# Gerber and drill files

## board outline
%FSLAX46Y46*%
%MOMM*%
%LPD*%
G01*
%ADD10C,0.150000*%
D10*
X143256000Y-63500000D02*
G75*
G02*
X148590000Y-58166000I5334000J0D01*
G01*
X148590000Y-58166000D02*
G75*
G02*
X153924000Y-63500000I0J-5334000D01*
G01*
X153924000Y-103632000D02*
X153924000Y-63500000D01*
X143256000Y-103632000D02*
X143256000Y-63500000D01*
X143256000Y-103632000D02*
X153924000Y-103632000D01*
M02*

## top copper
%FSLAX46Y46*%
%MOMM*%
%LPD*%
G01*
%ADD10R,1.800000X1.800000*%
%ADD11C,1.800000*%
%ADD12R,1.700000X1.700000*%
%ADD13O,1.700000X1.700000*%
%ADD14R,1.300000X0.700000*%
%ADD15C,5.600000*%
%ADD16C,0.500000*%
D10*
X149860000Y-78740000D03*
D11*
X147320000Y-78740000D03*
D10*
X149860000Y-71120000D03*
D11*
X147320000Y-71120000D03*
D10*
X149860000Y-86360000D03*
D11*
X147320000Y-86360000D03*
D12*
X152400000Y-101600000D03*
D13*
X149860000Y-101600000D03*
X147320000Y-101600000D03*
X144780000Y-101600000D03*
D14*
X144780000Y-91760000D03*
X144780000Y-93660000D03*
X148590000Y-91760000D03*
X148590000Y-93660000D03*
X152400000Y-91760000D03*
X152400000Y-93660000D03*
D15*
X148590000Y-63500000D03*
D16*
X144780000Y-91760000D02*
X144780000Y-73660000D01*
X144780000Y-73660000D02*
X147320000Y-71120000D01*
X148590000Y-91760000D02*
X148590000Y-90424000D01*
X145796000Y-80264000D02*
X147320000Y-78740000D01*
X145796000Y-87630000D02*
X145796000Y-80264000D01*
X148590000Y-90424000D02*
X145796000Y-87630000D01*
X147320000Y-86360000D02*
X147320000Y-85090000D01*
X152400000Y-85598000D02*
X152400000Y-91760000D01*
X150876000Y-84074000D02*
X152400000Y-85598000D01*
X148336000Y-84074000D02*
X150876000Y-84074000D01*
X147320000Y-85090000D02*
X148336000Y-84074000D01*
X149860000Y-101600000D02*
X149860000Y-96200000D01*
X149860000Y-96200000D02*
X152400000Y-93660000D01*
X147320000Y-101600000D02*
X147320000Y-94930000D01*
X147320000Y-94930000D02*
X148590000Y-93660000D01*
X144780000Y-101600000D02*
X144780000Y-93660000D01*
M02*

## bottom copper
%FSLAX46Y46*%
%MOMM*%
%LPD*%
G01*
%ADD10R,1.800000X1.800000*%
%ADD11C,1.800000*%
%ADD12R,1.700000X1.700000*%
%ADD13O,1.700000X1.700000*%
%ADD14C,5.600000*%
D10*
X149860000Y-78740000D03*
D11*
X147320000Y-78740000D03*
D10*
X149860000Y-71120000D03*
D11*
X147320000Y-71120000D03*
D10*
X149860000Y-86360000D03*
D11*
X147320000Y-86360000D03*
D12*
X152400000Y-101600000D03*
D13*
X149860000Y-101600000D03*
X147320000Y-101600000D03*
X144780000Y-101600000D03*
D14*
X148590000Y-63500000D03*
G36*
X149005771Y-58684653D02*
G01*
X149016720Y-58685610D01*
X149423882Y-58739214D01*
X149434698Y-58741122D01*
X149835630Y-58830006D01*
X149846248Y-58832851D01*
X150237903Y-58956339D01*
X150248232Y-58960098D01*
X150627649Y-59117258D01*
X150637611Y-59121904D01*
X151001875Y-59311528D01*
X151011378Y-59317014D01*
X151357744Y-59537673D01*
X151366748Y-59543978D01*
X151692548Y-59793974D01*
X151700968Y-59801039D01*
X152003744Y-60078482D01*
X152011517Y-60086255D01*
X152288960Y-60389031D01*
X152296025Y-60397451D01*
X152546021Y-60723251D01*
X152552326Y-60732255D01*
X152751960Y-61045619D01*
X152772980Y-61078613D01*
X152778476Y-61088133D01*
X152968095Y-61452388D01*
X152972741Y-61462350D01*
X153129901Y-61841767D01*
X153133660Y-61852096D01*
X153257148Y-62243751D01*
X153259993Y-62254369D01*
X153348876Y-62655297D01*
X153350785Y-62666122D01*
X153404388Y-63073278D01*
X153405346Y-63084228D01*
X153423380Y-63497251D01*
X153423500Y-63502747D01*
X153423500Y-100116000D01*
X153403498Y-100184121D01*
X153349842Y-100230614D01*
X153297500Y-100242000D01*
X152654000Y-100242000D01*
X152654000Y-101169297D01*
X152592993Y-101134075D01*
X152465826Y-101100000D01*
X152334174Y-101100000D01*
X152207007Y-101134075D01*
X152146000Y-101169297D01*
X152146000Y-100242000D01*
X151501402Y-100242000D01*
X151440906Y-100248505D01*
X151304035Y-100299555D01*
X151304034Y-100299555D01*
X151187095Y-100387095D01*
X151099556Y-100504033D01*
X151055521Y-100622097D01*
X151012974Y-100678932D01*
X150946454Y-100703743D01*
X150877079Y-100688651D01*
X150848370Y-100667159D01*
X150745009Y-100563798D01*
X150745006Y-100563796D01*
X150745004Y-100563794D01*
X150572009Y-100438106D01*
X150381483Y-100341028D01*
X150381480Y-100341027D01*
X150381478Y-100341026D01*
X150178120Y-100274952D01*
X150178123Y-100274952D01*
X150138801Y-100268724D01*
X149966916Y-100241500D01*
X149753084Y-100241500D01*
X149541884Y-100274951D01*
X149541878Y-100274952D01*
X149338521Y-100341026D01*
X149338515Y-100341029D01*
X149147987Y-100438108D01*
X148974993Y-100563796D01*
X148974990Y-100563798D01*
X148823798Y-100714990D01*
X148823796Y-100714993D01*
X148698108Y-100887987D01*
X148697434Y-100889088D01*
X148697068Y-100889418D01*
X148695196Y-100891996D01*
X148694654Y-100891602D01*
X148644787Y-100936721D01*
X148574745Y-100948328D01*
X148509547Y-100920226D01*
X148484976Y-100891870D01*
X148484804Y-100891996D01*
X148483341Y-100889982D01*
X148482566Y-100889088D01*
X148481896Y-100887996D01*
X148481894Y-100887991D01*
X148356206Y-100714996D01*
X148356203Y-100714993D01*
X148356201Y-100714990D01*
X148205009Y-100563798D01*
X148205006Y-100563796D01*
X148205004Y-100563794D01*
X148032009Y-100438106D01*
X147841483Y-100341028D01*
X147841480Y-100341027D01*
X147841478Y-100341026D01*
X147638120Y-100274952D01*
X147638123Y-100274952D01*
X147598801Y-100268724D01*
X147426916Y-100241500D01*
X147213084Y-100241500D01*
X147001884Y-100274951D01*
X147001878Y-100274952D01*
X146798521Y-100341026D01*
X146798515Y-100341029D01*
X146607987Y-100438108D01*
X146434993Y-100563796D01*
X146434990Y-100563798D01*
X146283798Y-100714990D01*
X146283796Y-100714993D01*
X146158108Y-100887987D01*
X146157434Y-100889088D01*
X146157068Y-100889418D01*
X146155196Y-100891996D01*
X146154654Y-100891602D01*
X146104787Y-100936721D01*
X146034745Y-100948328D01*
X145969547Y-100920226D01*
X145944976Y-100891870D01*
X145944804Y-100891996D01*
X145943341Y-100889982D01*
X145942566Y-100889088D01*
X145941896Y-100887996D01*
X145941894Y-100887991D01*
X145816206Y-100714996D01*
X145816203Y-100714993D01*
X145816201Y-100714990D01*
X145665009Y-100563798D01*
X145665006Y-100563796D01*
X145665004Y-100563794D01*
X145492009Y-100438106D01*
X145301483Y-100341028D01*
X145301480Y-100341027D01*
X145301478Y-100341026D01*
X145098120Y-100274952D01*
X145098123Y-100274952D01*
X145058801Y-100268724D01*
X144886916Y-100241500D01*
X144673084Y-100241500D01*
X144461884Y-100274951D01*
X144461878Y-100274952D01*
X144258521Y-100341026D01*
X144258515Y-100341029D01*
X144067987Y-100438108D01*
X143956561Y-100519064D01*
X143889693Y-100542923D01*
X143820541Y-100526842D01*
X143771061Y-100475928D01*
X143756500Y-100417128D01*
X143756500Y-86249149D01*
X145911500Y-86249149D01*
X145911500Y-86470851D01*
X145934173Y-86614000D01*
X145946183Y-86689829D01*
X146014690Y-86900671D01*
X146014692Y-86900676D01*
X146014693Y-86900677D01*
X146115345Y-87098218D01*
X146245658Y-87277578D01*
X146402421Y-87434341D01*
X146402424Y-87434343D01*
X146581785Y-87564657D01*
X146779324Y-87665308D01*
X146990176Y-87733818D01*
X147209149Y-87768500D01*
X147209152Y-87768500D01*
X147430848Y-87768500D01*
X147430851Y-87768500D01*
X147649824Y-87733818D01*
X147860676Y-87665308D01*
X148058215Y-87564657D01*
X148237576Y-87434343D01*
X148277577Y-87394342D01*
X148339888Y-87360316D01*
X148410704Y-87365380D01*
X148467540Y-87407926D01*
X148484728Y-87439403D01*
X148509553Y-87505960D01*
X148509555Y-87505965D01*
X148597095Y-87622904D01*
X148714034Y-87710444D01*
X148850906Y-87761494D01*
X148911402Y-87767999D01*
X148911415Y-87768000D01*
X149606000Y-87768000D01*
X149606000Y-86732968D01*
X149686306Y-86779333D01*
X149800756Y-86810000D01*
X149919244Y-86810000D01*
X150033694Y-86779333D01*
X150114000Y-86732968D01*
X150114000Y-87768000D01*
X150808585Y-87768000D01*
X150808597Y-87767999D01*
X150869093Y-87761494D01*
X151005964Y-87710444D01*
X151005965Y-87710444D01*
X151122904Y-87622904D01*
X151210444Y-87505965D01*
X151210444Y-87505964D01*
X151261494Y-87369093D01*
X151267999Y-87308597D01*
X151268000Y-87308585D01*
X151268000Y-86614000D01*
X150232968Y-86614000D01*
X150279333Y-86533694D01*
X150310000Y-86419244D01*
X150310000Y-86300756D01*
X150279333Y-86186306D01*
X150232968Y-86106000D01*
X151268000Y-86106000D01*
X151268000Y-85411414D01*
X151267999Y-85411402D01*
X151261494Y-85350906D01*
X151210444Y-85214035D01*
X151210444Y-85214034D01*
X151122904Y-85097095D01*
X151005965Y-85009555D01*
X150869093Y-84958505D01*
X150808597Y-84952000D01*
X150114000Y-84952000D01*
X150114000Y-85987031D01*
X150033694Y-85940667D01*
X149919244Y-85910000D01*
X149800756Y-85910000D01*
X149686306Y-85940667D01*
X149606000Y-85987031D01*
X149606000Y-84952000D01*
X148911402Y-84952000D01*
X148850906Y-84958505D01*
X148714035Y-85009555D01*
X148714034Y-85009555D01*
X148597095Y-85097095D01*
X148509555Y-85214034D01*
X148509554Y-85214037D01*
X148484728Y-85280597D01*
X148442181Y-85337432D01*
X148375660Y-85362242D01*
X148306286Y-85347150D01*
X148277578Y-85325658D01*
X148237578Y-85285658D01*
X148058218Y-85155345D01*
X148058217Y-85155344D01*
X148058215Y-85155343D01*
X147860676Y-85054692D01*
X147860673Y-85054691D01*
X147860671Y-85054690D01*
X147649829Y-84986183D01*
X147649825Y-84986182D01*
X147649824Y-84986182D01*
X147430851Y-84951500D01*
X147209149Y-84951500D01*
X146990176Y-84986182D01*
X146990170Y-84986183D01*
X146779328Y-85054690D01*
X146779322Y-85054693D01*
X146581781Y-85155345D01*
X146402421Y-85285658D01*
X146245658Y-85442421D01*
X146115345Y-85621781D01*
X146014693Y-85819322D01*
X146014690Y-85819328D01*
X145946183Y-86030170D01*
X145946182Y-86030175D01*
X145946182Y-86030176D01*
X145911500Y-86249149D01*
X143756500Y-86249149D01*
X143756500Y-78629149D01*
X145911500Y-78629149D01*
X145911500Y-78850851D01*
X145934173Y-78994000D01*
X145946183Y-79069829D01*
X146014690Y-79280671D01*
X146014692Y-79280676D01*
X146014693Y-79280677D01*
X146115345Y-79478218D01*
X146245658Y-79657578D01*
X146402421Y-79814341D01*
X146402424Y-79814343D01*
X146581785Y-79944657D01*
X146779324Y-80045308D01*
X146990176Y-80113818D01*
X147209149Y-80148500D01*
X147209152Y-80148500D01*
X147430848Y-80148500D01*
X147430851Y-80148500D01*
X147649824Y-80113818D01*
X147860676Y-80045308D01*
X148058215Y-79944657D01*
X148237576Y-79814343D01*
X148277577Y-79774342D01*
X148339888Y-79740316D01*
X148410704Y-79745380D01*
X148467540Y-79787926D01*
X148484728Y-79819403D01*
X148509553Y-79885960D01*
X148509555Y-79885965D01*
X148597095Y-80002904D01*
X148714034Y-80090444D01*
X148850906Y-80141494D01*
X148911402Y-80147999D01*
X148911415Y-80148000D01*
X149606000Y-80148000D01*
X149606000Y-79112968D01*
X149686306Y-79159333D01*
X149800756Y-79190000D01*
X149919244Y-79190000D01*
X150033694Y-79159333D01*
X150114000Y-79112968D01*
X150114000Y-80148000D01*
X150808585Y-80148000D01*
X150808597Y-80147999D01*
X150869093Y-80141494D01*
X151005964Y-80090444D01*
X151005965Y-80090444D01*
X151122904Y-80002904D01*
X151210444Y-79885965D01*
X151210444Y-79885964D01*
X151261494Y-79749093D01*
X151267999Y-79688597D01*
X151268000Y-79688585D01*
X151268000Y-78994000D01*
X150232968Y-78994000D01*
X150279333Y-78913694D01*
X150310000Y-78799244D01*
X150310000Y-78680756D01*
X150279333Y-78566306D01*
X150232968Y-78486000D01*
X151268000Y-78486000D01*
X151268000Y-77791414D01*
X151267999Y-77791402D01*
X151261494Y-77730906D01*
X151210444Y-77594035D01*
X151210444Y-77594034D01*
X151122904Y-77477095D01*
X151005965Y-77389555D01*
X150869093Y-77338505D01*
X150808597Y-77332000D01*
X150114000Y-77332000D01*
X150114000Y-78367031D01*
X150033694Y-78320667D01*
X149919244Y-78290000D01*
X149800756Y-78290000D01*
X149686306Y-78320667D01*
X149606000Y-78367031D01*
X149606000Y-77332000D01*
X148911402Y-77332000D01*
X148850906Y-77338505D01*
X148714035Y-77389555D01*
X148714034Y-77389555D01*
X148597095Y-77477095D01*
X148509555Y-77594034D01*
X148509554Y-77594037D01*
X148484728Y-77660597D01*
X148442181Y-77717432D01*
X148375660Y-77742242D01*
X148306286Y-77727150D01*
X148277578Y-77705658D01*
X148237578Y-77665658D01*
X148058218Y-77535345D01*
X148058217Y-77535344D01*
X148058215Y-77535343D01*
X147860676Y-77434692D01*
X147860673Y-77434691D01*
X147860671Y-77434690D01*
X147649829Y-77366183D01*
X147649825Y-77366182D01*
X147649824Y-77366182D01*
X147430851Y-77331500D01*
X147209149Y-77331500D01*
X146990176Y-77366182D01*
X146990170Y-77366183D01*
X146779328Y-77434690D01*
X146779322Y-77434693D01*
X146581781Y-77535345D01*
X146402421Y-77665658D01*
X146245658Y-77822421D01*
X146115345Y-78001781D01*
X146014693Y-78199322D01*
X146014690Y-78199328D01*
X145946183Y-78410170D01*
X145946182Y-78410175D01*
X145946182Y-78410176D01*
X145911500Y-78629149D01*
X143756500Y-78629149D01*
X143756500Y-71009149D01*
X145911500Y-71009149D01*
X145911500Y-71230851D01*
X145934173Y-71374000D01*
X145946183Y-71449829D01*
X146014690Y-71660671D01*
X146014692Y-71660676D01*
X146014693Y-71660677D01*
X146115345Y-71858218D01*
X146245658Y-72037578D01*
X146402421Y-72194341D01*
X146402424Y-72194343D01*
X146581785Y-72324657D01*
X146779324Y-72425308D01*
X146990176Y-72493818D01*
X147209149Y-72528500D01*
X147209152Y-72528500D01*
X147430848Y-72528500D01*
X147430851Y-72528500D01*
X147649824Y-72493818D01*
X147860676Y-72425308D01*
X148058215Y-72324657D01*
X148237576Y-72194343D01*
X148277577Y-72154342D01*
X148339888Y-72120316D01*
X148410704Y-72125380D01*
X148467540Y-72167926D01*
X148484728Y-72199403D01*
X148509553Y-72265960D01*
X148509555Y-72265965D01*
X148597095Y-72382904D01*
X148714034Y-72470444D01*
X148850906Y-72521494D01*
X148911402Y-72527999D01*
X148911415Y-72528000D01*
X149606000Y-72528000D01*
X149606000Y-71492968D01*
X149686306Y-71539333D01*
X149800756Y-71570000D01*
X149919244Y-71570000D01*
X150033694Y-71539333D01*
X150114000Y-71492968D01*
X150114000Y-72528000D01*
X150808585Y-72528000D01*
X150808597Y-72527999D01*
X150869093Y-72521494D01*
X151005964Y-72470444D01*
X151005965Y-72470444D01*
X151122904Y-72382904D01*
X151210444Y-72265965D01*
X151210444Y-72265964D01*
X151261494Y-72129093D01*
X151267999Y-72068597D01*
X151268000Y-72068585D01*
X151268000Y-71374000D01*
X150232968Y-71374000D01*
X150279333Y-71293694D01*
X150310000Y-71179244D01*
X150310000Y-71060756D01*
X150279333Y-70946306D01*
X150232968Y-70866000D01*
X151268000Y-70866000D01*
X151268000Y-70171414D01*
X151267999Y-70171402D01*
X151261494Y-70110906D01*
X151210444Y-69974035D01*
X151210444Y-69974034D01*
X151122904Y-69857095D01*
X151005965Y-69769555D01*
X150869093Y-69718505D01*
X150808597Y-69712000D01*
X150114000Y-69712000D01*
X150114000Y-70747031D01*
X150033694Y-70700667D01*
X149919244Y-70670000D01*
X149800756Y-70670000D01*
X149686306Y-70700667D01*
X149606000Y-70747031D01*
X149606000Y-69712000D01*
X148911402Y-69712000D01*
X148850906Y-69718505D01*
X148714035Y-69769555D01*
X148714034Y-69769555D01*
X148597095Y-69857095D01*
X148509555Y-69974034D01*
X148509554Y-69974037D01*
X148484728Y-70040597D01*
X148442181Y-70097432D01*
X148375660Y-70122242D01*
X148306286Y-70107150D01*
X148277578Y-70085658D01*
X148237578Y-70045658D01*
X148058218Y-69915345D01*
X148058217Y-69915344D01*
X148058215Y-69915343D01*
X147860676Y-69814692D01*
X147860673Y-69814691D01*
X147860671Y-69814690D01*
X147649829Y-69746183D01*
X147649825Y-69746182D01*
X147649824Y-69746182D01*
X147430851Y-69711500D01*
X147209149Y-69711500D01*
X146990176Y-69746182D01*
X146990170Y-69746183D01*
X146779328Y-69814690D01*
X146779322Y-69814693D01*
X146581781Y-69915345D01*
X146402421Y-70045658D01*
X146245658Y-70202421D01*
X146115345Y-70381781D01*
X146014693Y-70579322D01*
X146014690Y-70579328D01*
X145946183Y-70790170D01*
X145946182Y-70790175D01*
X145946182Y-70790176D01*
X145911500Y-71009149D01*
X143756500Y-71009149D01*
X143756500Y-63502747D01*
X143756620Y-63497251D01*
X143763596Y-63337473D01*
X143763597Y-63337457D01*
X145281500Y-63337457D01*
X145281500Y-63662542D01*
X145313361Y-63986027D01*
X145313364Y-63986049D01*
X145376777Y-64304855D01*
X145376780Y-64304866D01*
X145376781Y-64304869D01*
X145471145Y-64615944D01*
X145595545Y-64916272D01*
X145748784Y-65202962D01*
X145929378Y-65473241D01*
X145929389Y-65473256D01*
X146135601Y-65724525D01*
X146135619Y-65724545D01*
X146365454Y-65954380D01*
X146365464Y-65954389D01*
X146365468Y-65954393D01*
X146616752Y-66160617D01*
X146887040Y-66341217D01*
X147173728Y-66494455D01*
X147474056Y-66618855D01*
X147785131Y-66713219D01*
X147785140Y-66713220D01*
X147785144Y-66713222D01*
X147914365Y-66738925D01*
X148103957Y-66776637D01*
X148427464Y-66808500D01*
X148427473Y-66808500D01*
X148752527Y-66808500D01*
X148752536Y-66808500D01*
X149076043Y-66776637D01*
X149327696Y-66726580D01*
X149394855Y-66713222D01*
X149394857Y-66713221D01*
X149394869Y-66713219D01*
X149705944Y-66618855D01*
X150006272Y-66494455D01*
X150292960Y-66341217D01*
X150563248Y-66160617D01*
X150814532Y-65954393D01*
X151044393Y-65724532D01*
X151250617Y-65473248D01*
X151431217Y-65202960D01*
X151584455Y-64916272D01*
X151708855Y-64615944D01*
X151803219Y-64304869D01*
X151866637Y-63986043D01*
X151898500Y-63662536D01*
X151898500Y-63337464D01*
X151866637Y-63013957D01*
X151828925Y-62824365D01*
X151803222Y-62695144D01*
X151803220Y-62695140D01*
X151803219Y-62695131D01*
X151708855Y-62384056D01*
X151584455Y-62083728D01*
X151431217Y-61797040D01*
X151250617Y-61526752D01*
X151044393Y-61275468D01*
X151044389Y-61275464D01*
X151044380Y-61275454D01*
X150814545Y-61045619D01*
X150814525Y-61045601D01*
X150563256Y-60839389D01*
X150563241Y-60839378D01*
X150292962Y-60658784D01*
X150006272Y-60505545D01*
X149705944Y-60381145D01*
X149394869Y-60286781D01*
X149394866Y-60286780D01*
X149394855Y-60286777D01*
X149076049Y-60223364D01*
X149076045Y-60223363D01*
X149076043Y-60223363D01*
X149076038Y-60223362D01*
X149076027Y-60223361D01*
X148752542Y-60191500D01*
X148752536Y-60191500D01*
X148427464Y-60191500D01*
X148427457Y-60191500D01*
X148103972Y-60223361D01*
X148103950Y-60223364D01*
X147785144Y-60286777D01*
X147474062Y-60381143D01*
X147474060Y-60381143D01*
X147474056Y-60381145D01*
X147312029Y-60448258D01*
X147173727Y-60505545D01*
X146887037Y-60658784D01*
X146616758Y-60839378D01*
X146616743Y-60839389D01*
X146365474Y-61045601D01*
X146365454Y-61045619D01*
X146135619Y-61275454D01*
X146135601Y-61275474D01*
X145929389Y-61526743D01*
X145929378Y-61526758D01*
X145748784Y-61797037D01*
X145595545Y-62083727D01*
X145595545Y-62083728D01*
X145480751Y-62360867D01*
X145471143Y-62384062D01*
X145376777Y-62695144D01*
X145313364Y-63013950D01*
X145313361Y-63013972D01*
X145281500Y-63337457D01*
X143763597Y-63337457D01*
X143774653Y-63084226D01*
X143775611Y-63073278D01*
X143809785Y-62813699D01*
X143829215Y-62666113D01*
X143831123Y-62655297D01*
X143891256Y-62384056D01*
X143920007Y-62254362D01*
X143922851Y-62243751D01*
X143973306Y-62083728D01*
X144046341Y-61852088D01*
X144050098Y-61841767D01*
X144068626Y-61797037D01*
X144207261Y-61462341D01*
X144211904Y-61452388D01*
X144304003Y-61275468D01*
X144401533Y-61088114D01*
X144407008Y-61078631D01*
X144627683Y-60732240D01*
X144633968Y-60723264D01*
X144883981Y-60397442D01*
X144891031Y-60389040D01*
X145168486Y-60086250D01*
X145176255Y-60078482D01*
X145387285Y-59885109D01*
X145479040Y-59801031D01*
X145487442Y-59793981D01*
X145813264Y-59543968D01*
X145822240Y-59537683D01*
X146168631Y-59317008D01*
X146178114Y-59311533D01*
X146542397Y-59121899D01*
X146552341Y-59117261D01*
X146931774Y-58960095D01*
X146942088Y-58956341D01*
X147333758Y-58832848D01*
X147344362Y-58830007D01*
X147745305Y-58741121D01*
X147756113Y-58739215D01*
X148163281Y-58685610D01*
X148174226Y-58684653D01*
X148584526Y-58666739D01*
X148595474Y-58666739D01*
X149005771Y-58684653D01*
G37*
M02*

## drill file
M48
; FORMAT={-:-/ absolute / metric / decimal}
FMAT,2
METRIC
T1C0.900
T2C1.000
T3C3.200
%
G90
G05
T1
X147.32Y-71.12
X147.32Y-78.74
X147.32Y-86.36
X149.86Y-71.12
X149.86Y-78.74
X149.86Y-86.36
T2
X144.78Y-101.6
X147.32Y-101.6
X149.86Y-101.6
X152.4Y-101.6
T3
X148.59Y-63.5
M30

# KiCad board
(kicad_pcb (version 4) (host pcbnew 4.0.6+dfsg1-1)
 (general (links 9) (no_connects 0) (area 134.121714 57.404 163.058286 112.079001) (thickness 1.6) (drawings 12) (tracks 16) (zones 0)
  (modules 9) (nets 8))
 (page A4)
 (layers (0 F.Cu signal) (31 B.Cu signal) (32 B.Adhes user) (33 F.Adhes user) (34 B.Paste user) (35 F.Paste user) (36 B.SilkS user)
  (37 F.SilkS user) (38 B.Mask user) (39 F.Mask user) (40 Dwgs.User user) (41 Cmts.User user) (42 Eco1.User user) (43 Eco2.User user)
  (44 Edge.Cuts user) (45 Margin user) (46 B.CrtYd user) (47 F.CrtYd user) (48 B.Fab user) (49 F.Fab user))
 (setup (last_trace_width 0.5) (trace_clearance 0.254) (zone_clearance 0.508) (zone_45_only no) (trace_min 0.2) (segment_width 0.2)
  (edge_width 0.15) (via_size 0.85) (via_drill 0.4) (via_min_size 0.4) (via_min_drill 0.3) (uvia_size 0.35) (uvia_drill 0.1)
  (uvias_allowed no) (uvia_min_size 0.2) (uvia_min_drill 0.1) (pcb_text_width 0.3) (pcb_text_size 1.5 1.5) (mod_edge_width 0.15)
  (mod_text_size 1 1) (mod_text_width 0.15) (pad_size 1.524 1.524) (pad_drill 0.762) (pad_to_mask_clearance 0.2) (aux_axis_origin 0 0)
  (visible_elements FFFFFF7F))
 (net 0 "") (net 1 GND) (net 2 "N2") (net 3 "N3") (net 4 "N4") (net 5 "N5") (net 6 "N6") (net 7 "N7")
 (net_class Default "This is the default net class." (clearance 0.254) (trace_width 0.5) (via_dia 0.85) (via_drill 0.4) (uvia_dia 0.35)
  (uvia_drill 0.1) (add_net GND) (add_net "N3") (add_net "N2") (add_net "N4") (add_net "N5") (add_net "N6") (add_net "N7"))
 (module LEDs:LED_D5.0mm (layer F.Cu) (at 149.86 78.74 180)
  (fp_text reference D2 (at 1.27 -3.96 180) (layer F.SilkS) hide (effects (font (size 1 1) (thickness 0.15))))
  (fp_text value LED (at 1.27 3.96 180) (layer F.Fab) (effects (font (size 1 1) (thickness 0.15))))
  (pad 1 thru_hole rect (at 0 0 180) (size 1.8 1.8) (drill 0.9) (layers *.Cu *.Mask) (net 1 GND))
  (pad 2 thru_hole circle (at 2.54 0 180) (size 1.8 1.8) (drill 0.9) (layers *.Cu *.Mask) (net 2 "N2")))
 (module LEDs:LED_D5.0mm (layer F.Cu) (at 149.86 71.12 180)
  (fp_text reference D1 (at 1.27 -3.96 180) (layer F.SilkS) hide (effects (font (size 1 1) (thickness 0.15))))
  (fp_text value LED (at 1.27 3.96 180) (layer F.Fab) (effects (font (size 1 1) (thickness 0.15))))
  (pad 1 thru_hole rect (at 0 0 180) (size 1.8 1.8) (drill 0.9) (layers *.Cu *.Mask) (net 1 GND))
  (pad 2 thru_hole circle (at 2.54 0 180) (size 1.8 1.8) (drill 0.9) (layers *.Cu *.Mask) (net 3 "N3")))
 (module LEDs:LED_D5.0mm (layer F.Cu) (at 149.86 86.36 180)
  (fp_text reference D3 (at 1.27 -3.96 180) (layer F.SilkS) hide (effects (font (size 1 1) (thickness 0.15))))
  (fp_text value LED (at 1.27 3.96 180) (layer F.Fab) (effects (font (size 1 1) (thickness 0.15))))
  (pad 1 thru_hole rect (at 0 0 180) (size 1.8 1.8) (drill 0.9) (layers *.Cu *.Mask) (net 1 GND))
  (pad 2 thru_hole circle (at 2.54 0 180) (size 1.8 1.8) (drill 0.9) (layers *.Cu *.Mask) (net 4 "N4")))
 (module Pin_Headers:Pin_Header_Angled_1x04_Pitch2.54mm (layer F.Cu) (at 152.4 101.6 270)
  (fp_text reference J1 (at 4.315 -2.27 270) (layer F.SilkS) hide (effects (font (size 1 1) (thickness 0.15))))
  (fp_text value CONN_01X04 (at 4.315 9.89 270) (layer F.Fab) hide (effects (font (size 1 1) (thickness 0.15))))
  (pad 1 thru_hole rect (at 0 0 270) (size 1.7 1.7) (drill 1) (layers *.Cu *.Mask) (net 1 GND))
  (pad 2 thru_hole oval (at 0 2.54 270) (size 1.7 1.7) (drill 1) (layers *.Cu *.Mask) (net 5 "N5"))
  (pad 3 thru_hole oval (at 0 5.08 270) (size 1.7 1.7) (drill 1) (layers *.Cu *.Mask) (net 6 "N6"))
  (pad 4 thru_hole oval (at 0 7.62 270) (size 1.7 1.7) (drill 1) (layers *.Cu *.Mask) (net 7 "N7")))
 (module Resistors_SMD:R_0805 (layer F.Cu) (at 144.78 92.71 270)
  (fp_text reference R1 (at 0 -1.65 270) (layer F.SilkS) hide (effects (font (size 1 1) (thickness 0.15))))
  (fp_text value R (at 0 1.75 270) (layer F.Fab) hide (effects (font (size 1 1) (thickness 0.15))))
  (pad 1 smd rect (at -0.95 0 270) (size 0.7 1.3) (layers F.Cu F.Paste F.Mask) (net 3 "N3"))
  (pad 2 smd rect (at 0.95 0 270) (size 0.7 1.3) (layers F.Cu F.Paste F.Mask) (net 7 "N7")))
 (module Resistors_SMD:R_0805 (layer F.Cu) (at 148.59 92.71 270)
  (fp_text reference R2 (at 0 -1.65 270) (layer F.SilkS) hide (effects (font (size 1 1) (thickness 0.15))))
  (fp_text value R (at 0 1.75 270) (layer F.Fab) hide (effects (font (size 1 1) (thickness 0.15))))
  (pad 1 smd rect (at -0.95 0 270) (size 0.7 1.3) (layers F.Cu F.Paste F.Mask) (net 2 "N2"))
  (pad 2 smd rect (at 0.95 0 270) (size 0.7 1.3) (layers F.Cu F.Paste F.Mask) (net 6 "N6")))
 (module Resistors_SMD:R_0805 (layer F.Cu) (at 152.4 92.71 270)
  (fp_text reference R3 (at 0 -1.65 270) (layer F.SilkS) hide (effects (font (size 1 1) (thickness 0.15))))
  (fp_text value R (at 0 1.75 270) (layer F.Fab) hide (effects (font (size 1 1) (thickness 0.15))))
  (pad 1 smd rect (at -0.95 0 270) (size 0.7 1.3) (layers F.Cu F.Paste F.Mask) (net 4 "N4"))
  (pad 2 smd rect (at 0.95 0 270) (size 0.7 1.3) (layers F.Cu F.Paste F.Mask) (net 5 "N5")))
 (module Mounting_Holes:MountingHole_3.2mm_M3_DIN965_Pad (layer F.Cu) (at 148.59 63.5)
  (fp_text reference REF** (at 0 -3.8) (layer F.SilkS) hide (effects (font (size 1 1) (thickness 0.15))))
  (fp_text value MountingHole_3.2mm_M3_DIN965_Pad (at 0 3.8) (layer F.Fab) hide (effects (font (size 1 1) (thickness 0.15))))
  (pad 1 thru_hole circle (at 0 0) (size 5.6 5.6) (drill 3.2) (layers *.Cu *.Mask)))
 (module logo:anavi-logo (layer F.Cu) (at 144.526 88.138 90)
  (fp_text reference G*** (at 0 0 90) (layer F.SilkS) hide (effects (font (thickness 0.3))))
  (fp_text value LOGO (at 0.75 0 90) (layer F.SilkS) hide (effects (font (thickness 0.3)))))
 (gr_arc (start 148.59 63.5) (end 143.256 63.5) (angle 90) (layer Edge.Cuts) (width 0.15))
 (gr_arc (start 148.59 63.5) (end 148.59 58.166) (angle 90) (layer Edge.Cuts) (width 0.15))
 (gr_line (start 153.924 103.632) (end 153.924 63.5) (angle 90) (layer Edge.Cuts) (width 0.15))
 (gr_line (start 143.256 103.632) (end 143.256 63.5) (angle 90) (layer Edge.Cuts) (width 0.15))
 (gr_line (start 143.256 103.632) (end 153.924 103.632) (angle 90) (layer Edge.Cuts) (width 0.15))
 (segment (start 144.78 91.76) (end 144.78 73.66) (width 0.5) (layer F.Cu) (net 3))
 (segment (start 144.78 73.66) (end 147.32 71.12) (width 0.5) (layer F.Cu) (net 3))
 (segment (start 148.59 91.76) (end 148.59 90.424) (width 0.5) (layer F.Cu) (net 2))
 (segment (start 145.796 80.264) (end 147.32 78.74) (width 0.5) (layer F.Cu) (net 2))
 (segment (start 145.796 87.63) (end 145.796 80.264) (width 0.5) (layer F.Cu) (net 2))
 (segment (start 148.59 90.424) (end 145.796 87.63) (width 0.5) (layer F.Cu) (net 2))
 (segment (start 147.32 86.36) (end 147.32 85.09) (width 0.5) (layer F.Cu) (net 4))
 (segment (start 152.4 85.598) (end 152.4 91.76) (width 0.5) (layer F.Cu) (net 4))
 (segment (start 150.876 84.074) (end 152.4 85.598) (width 0.5) (layer F.Cu) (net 4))
 (segment (start 148.336 84.074) (end 150.876 84.074) (width 0.5) (layer F.Cu) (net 4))
 (segment (start 147.32 85.09) (end 148.336 84.074) (width 0.5) (layer F.Cu) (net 4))
 (segment (start 149.86 101.6) (end 149.86 96.2) (width 0.5) (layer F.Cu) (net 5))
 (segment (start 149.86 96.2) (end 152.4 93.66) (width 0.5) (layer F.Cu) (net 5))
 (segment (start 147.32 101.6) (end 147.32 94.93) (width 0.5) (layer F.Cu) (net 6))
 (segment (start 147.32 94.93) (end 148.59 93.66) (width 0.5) (layer F.Cu) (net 6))
 (segment (start 144.78 101.6) (end 144.78 93.66) (width 0.5) (layer F.Cu) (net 7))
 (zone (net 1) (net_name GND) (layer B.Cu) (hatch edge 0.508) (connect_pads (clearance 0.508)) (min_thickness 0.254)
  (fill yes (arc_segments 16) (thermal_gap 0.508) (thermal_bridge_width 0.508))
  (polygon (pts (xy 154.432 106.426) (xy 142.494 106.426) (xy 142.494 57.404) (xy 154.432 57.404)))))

